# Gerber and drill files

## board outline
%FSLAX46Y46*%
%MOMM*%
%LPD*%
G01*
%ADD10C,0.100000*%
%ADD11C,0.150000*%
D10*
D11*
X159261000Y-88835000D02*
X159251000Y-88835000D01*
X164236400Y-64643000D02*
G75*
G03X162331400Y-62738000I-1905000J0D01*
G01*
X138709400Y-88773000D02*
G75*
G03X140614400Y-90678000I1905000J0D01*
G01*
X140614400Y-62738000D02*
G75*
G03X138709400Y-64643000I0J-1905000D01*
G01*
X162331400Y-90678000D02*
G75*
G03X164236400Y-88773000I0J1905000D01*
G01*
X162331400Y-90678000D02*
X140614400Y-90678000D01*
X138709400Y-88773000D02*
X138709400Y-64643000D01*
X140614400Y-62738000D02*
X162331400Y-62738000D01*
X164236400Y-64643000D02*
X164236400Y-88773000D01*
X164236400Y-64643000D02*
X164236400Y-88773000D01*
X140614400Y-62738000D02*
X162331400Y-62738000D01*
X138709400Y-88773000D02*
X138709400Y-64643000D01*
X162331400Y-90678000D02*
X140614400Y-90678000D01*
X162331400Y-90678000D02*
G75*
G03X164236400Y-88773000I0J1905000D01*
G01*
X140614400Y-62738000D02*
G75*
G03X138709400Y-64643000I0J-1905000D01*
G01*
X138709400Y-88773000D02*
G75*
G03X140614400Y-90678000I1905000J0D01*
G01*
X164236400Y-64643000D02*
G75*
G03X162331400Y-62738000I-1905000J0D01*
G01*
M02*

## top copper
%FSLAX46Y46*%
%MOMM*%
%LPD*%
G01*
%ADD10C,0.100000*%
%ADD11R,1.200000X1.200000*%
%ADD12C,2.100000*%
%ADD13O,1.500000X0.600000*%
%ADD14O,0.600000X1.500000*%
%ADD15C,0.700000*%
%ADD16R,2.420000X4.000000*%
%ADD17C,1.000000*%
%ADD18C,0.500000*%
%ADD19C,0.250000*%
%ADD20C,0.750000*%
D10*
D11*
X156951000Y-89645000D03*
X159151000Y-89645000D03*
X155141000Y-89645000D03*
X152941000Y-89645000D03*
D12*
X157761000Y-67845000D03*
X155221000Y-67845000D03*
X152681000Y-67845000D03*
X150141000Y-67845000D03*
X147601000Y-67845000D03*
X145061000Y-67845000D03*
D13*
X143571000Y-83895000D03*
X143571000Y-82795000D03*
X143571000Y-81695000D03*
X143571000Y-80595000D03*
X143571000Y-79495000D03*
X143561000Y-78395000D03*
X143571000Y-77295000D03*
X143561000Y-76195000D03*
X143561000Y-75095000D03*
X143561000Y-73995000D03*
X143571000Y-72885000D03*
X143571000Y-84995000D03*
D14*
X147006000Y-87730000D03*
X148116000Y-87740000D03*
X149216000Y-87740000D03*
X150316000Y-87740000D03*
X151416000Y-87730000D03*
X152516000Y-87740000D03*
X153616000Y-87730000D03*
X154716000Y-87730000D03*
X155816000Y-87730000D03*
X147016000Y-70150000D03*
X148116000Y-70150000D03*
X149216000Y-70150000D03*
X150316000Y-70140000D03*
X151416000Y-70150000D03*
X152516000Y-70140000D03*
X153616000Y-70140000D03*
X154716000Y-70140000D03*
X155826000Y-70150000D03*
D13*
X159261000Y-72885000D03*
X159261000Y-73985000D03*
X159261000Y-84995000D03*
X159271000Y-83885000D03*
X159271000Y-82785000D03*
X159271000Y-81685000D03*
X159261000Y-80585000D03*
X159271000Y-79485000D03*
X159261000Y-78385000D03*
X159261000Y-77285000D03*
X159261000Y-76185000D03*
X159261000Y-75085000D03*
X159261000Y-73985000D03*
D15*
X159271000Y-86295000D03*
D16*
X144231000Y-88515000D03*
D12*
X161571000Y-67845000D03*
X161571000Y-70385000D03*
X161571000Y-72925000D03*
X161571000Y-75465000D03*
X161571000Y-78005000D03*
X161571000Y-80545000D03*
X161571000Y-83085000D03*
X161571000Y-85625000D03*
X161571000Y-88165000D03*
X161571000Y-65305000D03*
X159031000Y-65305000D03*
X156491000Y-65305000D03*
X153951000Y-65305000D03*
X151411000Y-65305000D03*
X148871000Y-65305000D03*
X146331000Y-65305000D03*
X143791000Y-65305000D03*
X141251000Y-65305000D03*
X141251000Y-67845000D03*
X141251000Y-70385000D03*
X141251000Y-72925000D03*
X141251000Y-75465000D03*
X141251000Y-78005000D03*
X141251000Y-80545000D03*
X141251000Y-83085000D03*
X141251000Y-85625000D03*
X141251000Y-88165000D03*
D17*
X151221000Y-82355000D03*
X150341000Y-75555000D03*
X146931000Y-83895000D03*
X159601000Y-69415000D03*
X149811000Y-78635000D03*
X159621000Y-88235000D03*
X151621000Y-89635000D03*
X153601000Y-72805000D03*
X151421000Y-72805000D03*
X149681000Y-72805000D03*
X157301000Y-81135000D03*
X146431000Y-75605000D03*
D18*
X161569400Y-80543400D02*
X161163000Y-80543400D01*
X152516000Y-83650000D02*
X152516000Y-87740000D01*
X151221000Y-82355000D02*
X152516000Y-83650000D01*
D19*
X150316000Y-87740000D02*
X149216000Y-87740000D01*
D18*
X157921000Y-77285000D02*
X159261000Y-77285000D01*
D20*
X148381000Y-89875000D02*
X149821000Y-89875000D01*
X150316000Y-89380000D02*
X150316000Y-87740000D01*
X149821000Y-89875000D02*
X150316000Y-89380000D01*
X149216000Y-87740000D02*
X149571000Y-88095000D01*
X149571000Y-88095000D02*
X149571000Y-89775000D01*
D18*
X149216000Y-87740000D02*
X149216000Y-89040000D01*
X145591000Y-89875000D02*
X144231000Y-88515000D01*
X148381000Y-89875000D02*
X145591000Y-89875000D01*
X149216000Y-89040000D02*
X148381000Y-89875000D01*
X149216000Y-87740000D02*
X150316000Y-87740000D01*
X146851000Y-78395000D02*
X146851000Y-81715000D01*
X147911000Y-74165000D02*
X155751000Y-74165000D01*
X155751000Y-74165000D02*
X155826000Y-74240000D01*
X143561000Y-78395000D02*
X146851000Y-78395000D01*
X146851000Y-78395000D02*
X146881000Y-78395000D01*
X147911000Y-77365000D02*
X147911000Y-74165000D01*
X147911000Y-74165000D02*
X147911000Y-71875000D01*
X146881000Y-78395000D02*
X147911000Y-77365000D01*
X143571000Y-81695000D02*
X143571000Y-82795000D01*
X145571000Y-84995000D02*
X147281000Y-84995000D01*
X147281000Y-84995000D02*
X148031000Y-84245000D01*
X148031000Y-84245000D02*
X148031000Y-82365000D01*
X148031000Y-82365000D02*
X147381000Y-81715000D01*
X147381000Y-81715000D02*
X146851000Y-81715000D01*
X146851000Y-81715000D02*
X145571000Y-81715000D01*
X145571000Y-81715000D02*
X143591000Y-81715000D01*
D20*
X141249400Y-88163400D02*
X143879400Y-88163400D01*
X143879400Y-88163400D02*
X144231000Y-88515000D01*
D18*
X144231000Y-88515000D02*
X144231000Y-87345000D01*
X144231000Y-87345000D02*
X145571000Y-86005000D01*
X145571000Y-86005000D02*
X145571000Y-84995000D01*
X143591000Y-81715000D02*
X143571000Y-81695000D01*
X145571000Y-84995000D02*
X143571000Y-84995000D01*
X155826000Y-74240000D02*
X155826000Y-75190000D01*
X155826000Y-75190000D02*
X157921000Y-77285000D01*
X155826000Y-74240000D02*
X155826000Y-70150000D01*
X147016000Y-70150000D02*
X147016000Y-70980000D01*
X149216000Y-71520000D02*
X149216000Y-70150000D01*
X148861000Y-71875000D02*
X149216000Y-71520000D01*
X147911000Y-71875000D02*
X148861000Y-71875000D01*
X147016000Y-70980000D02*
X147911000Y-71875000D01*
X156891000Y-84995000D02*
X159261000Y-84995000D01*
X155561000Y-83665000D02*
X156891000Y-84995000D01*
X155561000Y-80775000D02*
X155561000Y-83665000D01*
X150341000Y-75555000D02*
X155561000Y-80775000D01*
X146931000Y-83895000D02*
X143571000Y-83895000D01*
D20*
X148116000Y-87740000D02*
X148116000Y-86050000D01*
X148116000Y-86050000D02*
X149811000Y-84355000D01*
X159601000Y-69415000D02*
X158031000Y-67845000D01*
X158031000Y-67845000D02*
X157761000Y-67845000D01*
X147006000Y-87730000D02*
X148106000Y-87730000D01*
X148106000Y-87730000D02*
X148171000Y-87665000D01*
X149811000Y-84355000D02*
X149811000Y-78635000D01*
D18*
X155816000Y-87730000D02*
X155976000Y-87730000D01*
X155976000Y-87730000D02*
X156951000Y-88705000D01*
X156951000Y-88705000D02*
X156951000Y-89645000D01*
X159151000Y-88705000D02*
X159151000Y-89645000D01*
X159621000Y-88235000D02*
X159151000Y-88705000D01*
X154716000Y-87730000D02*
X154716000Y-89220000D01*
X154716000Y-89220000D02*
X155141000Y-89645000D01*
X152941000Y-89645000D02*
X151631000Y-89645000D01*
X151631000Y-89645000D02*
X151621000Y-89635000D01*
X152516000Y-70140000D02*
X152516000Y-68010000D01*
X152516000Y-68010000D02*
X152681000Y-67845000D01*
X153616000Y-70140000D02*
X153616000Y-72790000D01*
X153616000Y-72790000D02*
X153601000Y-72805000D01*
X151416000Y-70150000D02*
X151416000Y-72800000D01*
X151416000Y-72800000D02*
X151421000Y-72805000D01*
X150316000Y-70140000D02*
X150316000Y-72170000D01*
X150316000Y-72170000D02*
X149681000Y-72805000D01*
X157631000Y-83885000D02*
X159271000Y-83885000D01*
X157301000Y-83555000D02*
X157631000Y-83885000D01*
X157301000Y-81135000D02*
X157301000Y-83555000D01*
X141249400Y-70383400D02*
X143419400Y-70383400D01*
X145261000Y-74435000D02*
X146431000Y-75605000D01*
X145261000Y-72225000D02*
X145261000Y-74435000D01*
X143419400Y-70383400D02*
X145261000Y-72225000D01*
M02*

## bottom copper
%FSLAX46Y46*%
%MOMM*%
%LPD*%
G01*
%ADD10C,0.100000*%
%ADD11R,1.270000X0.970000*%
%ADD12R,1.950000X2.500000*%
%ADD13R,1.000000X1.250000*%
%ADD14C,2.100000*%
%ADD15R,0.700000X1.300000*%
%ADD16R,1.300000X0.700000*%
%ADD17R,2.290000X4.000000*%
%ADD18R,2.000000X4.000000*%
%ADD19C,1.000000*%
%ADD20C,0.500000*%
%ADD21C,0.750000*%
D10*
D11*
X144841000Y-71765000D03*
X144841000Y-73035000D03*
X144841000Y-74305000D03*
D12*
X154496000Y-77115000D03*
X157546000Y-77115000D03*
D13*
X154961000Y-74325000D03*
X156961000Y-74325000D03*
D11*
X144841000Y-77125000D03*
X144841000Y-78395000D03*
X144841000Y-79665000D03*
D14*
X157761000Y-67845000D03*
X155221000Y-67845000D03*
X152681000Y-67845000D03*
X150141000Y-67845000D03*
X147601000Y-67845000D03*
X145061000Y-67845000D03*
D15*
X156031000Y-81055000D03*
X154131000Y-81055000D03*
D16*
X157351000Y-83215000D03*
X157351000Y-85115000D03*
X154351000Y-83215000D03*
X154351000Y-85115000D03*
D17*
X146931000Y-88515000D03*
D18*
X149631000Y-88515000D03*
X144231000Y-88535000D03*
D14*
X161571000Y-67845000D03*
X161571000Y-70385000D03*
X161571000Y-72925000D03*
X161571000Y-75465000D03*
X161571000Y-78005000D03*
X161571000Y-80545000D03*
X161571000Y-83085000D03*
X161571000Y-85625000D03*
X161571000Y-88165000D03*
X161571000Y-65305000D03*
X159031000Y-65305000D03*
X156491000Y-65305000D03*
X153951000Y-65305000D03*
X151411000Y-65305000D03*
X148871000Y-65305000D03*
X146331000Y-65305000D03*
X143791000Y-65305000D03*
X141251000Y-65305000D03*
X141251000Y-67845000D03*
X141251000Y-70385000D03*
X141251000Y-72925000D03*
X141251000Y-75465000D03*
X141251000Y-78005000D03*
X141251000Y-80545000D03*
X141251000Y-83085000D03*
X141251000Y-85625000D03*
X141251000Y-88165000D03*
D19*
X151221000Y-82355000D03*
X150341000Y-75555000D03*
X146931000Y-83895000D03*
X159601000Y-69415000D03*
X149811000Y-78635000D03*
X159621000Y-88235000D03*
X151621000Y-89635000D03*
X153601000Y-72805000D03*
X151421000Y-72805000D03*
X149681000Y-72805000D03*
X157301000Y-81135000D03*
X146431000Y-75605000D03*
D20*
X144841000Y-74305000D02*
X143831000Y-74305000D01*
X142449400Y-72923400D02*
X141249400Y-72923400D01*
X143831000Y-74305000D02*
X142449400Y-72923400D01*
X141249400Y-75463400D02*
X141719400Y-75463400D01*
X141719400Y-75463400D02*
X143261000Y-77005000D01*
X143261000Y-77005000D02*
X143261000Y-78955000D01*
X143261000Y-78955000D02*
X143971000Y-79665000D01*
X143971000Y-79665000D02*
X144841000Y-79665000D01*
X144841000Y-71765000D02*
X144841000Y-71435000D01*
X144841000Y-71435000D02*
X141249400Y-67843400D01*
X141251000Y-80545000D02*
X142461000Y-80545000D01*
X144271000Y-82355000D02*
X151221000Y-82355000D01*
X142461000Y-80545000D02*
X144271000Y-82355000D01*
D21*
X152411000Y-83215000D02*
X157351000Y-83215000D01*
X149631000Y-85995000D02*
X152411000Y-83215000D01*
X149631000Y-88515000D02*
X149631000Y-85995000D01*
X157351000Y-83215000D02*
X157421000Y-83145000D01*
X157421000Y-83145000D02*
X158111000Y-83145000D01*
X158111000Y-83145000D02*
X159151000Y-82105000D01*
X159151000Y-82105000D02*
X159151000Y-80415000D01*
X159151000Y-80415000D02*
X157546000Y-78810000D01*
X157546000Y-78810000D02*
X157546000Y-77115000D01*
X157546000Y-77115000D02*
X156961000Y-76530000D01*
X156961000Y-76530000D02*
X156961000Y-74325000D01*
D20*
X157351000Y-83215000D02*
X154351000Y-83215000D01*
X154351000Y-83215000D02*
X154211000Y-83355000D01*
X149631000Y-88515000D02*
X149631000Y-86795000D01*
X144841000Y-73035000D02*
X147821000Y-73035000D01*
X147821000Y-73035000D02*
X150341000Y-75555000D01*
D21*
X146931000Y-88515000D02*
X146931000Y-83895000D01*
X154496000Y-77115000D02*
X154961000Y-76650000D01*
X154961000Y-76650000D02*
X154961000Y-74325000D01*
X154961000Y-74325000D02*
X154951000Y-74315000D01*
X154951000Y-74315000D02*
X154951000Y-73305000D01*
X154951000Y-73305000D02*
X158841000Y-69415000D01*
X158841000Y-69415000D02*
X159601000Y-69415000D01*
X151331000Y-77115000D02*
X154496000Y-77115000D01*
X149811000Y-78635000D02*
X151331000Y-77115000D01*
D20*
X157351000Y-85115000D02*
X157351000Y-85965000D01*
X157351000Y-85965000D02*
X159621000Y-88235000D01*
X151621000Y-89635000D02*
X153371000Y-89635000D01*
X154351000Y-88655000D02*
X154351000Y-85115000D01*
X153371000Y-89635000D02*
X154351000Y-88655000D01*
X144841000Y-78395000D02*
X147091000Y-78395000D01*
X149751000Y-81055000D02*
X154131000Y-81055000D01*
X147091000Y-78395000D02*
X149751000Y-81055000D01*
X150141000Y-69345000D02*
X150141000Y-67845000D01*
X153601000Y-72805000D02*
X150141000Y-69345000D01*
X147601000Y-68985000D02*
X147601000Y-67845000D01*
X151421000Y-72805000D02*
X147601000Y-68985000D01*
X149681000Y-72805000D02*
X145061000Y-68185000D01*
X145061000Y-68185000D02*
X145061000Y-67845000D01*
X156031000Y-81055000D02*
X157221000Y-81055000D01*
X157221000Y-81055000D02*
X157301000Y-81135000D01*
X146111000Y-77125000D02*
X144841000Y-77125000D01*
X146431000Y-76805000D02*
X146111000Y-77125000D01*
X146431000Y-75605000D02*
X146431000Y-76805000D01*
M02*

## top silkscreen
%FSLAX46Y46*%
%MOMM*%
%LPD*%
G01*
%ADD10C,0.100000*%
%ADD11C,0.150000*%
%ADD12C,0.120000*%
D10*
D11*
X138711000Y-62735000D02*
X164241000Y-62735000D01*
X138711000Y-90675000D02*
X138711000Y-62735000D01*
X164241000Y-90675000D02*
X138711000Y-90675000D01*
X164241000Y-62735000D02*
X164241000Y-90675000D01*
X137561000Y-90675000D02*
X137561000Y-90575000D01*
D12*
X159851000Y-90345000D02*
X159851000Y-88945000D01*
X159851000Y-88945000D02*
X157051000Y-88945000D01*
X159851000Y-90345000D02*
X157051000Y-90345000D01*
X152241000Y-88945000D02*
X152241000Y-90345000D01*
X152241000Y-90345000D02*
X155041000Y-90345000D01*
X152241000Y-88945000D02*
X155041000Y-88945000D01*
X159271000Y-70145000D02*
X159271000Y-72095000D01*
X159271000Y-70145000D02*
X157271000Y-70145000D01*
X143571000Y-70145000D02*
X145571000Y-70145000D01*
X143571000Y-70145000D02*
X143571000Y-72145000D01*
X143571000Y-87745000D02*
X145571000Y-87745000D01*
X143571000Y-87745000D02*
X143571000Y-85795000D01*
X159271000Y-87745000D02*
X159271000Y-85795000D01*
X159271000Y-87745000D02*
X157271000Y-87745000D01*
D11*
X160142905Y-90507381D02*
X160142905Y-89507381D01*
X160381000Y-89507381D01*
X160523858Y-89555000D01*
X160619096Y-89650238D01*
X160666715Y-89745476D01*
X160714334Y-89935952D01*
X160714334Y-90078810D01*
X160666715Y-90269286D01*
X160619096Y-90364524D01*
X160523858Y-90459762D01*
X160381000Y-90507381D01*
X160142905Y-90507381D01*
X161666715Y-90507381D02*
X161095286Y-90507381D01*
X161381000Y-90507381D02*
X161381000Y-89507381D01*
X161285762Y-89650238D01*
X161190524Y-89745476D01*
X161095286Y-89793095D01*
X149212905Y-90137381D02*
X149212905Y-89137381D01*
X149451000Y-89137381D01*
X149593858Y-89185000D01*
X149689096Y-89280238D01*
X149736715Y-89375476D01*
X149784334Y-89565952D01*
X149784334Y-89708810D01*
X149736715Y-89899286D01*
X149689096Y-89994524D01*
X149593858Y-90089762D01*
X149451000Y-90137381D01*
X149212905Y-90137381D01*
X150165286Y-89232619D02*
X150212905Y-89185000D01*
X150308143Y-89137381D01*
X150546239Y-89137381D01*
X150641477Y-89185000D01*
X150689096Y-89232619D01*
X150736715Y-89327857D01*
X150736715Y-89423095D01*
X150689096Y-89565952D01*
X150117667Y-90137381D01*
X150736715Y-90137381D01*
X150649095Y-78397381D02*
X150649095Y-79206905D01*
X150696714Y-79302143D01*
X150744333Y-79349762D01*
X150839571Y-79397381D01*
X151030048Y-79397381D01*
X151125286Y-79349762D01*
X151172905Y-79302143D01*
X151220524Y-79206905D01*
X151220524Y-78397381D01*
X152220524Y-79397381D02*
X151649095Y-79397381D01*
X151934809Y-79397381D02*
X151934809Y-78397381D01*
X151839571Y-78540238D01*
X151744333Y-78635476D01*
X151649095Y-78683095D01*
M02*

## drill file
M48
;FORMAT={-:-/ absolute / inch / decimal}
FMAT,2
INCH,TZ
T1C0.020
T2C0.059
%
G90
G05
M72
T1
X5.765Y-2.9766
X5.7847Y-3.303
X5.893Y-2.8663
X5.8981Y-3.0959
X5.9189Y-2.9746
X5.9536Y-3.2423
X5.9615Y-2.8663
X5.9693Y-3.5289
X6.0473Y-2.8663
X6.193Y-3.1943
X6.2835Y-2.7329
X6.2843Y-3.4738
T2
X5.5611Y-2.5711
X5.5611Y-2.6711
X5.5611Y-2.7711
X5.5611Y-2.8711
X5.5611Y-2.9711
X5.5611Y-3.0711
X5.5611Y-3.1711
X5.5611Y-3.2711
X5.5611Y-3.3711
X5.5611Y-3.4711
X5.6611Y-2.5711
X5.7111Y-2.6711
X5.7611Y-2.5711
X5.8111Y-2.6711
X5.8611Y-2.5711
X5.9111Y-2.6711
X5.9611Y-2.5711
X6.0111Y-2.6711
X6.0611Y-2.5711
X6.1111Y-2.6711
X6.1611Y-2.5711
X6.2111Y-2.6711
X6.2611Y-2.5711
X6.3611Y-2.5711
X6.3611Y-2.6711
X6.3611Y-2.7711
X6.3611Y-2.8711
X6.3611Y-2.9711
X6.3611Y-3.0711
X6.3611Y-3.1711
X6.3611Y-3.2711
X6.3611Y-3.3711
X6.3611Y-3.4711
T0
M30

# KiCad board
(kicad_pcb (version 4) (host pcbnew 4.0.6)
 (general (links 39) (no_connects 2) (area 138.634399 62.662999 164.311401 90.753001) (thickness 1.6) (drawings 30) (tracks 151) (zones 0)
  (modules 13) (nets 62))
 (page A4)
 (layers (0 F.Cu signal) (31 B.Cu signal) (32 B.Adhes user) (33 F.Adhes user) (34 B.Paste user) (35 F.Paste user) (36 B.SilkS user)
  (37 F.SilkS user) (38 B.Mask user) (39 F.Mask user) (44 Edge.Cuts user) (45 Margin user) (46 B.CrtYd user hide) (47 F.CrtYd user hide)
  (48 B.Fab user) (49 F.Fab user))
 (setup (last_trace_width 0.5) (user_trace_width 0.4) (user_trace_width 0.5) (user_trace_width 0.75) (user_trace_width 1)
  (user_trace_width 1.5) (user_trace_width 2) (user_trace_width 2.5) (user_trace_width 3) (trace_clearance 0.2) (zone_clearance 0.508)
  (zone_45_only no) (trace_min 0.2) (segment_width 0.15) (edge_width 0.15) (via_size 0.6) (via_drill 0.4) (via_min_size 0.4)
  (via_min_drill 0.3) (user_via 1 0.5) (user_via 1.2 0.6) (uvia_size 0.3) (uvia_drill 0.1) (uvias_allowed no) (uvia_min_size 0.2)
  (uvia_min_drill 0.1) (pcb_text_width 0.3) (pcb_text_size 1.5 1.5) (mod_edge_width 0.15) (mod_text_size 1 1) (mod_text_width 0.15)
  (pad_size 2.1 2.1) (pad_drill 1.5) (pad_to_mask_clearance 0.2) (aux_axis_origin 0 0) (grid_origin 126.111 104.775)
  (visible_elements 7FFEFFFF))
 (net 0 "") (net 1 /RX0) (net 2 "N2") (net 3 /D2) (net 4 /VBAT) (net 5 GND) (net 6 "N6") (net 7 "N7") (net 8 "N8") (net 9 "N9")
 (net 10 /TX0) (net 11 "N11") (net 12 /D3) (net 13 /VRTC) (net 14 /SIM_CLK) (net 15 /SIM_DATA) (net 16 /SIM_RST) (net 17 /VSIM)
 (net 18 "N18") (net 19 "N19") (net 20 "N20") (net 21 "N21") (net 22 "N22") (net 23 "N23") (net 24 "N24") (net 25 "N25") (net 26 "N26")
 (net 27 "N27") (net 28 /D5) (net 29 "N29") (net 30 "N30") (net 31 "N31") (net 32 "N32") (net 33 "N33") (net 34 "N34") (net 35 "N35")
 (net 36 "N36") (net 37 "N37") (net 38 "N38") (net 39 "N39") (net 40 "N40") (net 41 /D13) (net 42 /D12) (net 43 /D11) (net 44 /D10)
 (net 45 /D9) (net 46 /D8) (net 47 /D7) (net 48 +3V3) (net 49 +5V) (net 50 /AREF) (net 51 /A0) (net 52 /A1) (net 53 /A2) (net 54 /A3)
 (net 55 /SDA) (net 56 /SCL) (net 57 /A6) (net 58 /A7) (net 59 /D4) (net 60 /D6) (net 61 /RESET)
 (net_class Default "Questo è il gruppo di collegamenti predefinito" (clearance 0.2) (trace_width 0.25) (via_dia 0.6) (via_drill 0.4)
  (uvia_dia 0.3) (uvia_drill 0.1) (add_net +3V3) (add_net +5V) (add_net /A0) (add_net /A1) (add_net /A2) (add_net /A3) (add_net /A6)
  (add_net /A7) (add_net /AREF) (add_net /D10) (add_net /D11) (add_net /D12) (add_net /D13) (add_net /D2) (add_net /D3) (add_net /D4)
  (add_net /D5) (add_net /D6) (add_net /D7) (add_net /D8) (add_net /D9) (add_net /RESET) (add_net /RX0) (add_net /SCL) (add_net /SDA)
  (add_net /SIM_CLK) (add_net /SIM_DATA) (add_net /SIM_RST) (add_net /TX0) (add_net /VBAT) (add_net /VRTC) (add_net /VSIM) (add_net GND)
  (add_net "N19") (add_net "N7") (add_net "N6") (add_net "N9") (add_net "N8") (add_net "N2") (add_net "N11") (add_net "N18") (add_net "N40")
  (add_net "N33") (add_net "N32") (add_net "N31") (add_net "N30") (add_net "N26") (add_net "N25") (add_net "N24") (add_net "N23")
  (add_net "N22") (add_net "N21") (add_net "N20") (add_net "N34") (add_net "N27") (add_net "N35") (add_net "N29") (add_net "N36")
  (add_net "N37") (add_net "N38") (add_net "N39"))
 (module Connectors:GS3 (layer B.Cu) (at 144.841 73.035 180)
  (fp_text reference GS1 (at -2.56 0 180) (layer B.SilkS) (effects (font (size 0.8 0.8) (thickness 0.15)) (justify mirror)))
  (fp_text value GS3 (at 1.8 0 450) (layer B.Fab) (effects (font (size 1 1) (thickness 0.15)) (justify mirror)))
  (pad 1 smd rect (at 0 1.27 180) (size 1.27 0.97) (layers B.Cu B.Paste B.Mask) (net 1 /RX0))
  (pad 2 smd rect (at 0 0 180) (size 1.27 0.97) (layers B.Cu B.Paste B.Mask) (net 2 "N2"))
  (pad 3 smd rect (at 0 -1.27 180) (size 1.27 0.97) (layers B.Cu B.Paste B.Mask) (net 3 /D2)))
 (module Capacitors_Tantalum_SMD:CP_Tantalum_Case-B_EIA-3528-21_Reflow (layer B.Cu) (at 156.021 77.115)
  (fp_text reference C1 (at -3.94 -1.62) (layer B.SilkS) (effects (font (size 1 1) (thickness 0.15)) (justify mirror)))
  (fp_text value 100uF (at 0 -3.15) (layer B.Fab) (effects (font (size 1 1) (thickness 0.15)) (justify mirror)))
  (pad 1 smd rect (at -1.525 0) (size 1.95 2.5) (layers B.Cu B.Paste B.Mask) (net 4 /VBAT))
  (pad 2 smd rect (at 1.525 0) (size 1.95 2.5) (layers B.Cu B.Paste B.Mask) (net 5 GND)))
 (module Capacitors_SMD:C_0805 (layer B.Cu) (at 155.961 74.325)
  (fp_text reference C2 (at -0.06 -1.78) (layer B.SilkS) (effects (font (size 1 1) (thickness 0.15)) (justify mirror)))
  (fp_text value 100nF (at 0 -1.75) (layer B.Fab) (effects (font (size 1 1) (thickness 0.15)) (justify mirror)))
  (pad 1 smd rect (at -1 0) (size 1 1.25) (layers B.Cu B.Paste B.Mask) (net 4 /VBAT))
  (pad 2 smd rect (at 1 0) (size 1 1.25) (layers B.Cu B.Paste B.Mask) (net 5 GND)))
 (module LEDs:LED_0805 (layer F.Cu) (at 158.051 89.645 180)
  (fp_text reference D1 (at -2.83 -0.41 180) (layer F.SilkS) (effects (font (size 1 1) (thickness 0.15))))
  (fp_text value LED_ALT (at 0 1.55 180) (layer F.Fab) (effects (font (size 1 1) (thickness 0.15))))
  (fp_line (start -1.8 -0.7) (end -1.8 0.7) (layer F.SilkS) (width 0.12))
  (fp_line (start -1.8 0.7) (end 1 0.7) (layer F.SilkS) (width 0.12))
  (fp_line (start -1.8 -0.7) (end 1 -0.7) (layer F.SilkS) (width 0.12))
  (pad 2 smd rect (at 1.1 0) (size 1.2 1.2) (layers F.Cu F.Paste F.Mask) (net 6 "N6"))
  (pad 1 smd rect (at -1.1 0) (size 1.2 1.2) (layers F.Cu F.Paste F.Mask) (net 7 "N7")))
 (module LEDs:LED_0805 (layer F.Cu) (at 154.041 89.645)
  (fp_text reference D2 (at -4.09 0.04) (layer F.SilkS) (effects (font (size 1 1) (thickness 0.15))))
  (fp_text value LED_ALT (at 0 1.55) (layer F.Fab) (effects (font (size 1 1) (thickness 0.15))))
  (fp_line (start -1.8 -0.7) (end -1.8 0.7) (layer F.SilkS) (width 0.12))
  (fp_line (start -1.8 0.7) (end 1 0.7) (layer F.SilkS) (width 0.12))
  (fp_line (start -1.8 -0.7) (end 1 -0.7) (layer F.SilkS) (width 0.12))
  (pad 2 smd rect (at 1.1 0 180) (size 1.2 1.2) (layers F.Cu F.Paste F.Mask) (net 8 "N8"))
  (pad 1 smd rect (at -1.1 0 180) (size 1.2 1.2) (layers F.Cu F.Paste F.Mask) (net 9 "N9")))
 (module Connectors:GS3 (layer B.Cu) (at 144.841 78.395 180)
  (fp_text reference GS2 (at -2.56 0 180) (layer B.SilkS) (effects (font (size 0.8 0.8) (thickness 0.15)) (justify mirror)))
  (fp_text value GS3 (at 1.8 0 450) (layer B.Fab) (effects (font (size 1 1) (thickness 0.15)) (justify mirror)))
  (pad 1 smd rect (at 0 1.27 180) (size 1.27 0.97) (layers B.Cu B.Paste B.Mask) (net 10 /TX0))
  (pad 2 smd rect (at 0 0 180) (size 1.27 0.97) (layers B.Cu B.Paste B.Mask) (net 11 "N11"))
  (pad 3 smd rect (at 0 -1.27 180) (size 1.27 0.97) (layers B.Cu B.Paste B.Mask) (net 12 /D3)))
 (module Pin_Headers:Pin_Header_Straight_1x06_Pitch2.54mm (layer B.Cu) (at 157.761 67.845 90)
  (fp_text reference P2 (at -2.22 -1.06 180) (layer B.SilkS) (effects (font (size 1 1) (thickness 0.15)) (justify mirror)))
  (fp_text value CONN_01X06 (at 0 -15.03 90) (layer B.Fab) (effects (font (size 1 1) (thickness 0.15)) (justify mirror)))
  (pad 1 thru_hole circle (at 0 0 90) (size 2.1 2.1) (drill 1.5) (layers *.Cu *.Mask) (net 4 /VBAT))
  (pad 2 thru_hole circle (at 0 -2.54 90) (size 2.1 2.1) (drill 1.5) (layers *.Cu *.Mask) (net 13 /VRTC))
  (pad 3 thru_hole circle (at 0 -5.08 90) (size 2.1 2.1) (drill 1.5) (layers *.Cu *.Mask) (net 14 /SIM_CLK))
  (pad 4 thru_hole circle (at 0 -7.62 90) (size 2.1 2.1) (drill 1.5) (layers *.Cu *.Mask) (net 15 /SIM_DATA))
  (pad 5 thru_hole circle (at 0 -10.16 90) (size 2.1 2.1) (drill 1.5) (layers *.Cu *.Mask) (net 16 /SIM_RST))
  (pad 6 thru_hole circle (at 0 -12.7 90) (size 2.1 2.1) (drill 1.5) (layers *.Cu *.Mask) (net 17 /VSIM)))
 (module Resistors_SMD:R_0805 (layer B.Cu) (at 155.081 81.055 180)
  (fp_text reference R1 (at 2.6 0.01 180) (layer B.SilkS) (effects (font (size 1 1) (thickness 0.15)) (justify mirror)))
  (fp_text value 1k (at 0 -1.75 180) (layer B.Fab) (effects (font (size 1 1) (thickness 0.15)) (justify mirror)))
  (pad 1 smd rect (at -0.95 0 180) (size 0.7 1.3) (layers B.Cu B.Paste B.Mask) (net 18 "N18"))
  (pad 2 smd rect (at 0.95 0 180) (size 0.7 1.3) (layers B.Cu B.Paste B.Mask) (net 11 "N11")))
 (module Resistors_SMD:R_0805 (layer B.Cu) (at 157.351 84.165 270)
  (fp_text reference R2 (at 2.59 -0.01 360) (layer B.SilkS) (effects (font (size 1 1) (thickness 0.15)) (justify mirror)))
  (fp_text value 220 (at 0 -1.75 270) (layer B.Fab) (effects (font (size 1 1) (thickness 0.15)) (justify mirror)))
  (pad 1 smd rect (at -0.95 0 270) (size 0.7 1.3) (layers B.Cu B.Paste B.Mask) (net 5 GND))
  (pad 2 smd rect (at 0.95 0 270) (size 0.7 1.3) (layers B.Cu B.Paste B.Mask) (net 7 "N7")))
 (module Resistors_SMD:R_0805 (layer B.Cu) (at 154.351 84.165 270)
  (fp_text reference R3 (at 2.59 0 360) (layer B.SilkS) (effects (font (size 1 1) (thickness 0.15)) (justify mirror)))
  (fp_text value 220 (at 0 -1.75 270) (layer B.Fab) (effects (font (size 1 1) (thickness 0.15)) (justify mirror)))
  (pad 1 smd rect (at -0.95 0 270) (size 0.7 1.3) (layers B.Cu B.Paste B.Mask) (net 5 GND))
  (pad 2 smd rect (at 0.95 0 270) (size 0.7 1.3) (layers B.Cu B.Paste B.Mask) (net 9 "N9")))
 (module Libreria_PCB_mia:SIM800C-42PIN (layer F.Cu) (at 151.421 78.945 180)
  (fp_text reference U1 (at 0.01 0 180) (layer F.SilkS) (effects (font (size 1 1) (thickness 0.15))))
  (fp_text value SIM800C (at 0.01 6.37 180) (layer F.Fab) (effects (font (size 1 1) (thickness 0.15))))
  (fp_line (start -7.85 8.8) (end -7.85 6.85) (layer F.SilkS) (width 0.12))
  (fp_line (start -7.85 8.8) (end -5.85 8.8) (layer F.SilkS) (width 0.12))
  (fp_line (start 7.85 8.8) (end 5.85 8.8) (layer F.SilkS) (width 0.12))
  (fp_line (start 7.85 8.8) (end 7.85 6.8) (layer F.SilkS) (width 0.12))
  (fp_line (start 7.85 -8.8) (end 5.85 -8.8) (layer F.SilkS) (width 0.12))
  (fp_line (start 7.85 -8.8) (end 7.85 -6.85) (layer F.SilkS) (width 0.12))
  (fp_line (start -7.85 -8.8) (end -7.85 -6.85) (layer F.SilkS) (width 0.12))
  (fp_line (start -7.85 -8.8) (end -5.85 -8.8) (layer F.SilkS) (width 0.12))
  (pad "" smd circle (at -7.85 -7.35 90) (size 0.7 0.7) (layers F.SilkS))
  (pad 32 smd oval (at 7.85 -4.95) (size 1.5 0.6) (layers F.Cu F.Paste F.Mask) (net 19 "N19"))
  (pad 31 smd oval (at 7.85 -3.85) (size 1.5 0.6) (layers F.Cu F.Paste F.Mask) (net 5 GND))
  (pad 30 smd oval (at 7.85 -2.75) (size 1.5 0.6) (layers F.Cu F.Paste F.Mask) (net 5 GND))
  (pad 29 smd oval (at 7.85 -1.65) (size 1.5 0.6) (layers F.Cu F.Paste F.Mask) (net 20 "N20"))
  (pad 28 smd oval (at 7.85 -0.55) (size 1.5 0.6) (layers F.Cu F.Paste F.Mask) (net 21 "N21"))
  (pad 27 smd oval (at 7.86 0.55) (size 1.5 0.6) (layers F.Cu F.Paste F.Mask) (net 5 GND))
  (pad 26 smd oval (at 7.85 1.65) (size 1.5 0.6) (layers F.Cu F.Paste F.Mask) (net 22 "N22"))
  (pad 25 smd oval (at 7.86 2.75) (size 1.5 0.6) (layers F.Cu F.Paste F.Mask) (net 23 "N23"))
  (pad 24 smd oval (at 7.86 3.85) (size 1.5 0.6) (layers F.Cu F.Paste F.Mask) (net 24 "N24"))
  (pad 23 smd oval (at 7.86 4.95) (size 1.5 0.6) (layers F.Cu F.Paste F.Mask) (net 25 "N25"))
  (pad 22 smd oval (at 7.85 6.06) (size 1.5 0.6) (layers F.Cu F.Paste F.Mask) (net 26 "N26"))
  (pad 33 smd oval (at 7.85 -6.05) (size 1.5 0.6) (layers F.Cu F.Paste F.Mask) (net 5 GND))
  (pad 34 smd oval (at 4.415 -8.785 90) (size 1.5 0.6) (layers F.Cu F.Paste F.Mask) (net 4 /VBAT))
  (pad 35 smd oval (at 3.305 -8.795 90) (size 1.5 0.6) (layers F.Cu F.Paste F.Mask) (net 4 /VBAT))
  (pad 36 smd oval (at 2.205 -8.795 90) (size 1.5 0.6) (layers F.Cu F.Paste F.Mask) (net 5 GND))
  (pad 37 smd oval (at 1.105 -8.795 90) (size 1.5 0.6) (layers F.Cu F.Paste F.Mask) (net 5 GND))
  (pad 38 smd oval (at 0.005 -8.785 90) (size 1.5 0.6) (layers F.Cu F.Paste F.Mask) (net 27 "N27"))
  (pad 39 smd oval (at -1.095 -8.795 90) (size 1.5 0.6) (layers F.Cu F.Paste F.Mask) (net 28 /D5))
  (pad 40 smd oval (at -2.195 -8.785 90) (size 1.5 0.6) (layers F.Cu F.Paste F.Mask) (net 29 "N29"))
  (pad 41 smd oval (at -3.295 -8.785 90) (size 1.5 0.6) (layers F.Cu F.Paste F.Mask) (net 8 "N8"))
  (pad 42 smd oval (at -4.395 -8.785 90) (size 1.5 0.6) (layers F.Cu F.Paste F.Mask) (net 6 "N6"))
  (pad 21 smd oval (at 4.405 8.795 270) (size 1.5 0.6) (layers F.Cu F.Paste F.Mask) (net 5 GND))
  (pad 20 smd oval (at 3.305 8.795 270) (size 1.5 0.6) (layers F.Cu F.Paste F.Mask) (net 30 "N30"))
  (pad 19 smd oval (at 2.205 8.795 270) (size 1.5 0.6) (layers F.Cu F.Paste F.Mask) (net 5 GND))
  (pad 18 smd oval (at 1.105 8.805 270) (size 1.5 0.6) (layers F.Cu F.Paste F.Mask) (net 17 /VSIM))
  (pad 17 smd oval (at 0.005 8.795 270) (size 1.5 0.6) (layers F.Cu F.Paste F.Mask) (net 16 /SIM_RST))
  (pad 16 smd oval (at -1.095 8.805 270) (size 1.5 0.6) (layers F.Cu F.Paste F.Mask) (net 14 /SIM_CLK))
  (pad 15 smd oval (at -2.195 8.805 270) (size 1.5 0.6) (layers F.Cu F.Paste F.Mask) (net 15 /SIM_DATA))
  (pad 14 smd oval (at -3.295 8.805 270) (size 1.5 0.6) (layers F.Cu F.Paste F.Mask) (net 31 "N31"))
  (pad 13 smd oval (at -4.405 8.795 270) (size 1.5 0.6) (layers F.Cu F.Paste F.Mask) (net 5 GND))
  (pad 12 smd oval (at -7.84 6.06 180) (size 1.5 0.6) (layers F.Cu F.Paste F.Mask) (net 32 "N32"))
  (pad 11 smd oval (at -7.84 4.96 180) (size 1.5 0.6) (layers F.Cu F.Paste F.Mask) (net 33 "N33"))
  (pad 1 smd oval (at -7.84 -6.05 180) (size 1.5 0.6) (layers F.Cu F.Paste F.Mask) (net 2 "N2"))
  (pad 2 smd oval (at -7.85 -4.94 180) (size 1.5 0.6) (layers F.Cu F.Paste F.Mask) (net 18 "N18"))
  (pad 3 smd oval (at -7.85 -3.84 180) (size 1.5 0.6) (layers F.Cu F.Paste F.Mask) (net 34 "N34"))
  (pad 4 smd oval (at -7.85 -2.74 180) (size 1.5 0.6) (layers F.Cu F.Paste F.Mask) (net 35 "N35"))
  (pad 5 smd oval (at -7.84 -1.64 180) (size 1.5 0.6) (layers F.Cu F.Paste F.Mask) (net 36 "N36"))
  (pad 6 smd oval (at -7.85 -0.54 180) (size 1.5 0.6) (layers F.Cu F.Paste F.Mask) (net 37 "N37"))
  (pad 7 smd oval (at -7.84 0.56 180) (size 1.5 0.6) (layers F.Cu F.Paste F.Mask) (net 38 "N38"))
  (pad 8 smd oval (at -7.84 1.66 180) (size 1.5 0.6) (layers F.Cu F.Paste F.Mask) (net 5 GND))
  (pad 9 smd oval (at -7.84 2.76 180) (size 1.5 0.6) (layers F.Cu F.Paste F.Mask) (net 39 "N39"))
  (pad 10 smd oval (at -7.84 3.86 180) (size 1.5 0.6) (layers F.Cu F.Paste F.Mask) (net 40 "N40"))
  (pad 11 smd oval (at -7.84 4.96 180) (size 1.5 0.6) (layers F.Cu F.Paste F.Mask) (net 33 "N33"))
  (pad "" smd circle (at -7.85 -7.35 90) (size 0.7 0.7) (layers F.Cu F.Paste F.Mask)))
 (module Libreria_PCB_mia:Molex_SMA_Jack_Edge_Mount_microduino (layer B.Cu) (at 146.931 88.535 90)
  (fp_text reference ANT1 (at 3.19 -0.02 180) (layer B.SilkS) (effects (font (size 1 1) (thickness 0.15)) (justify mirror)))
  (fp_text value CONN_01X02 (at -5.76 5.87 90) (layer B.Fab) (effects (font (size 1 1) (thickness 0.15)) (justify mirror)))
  (pad 1 smd rect (at 0.02 0 90) (size 4 2.29) (layers B.Cu B.Paste B.Mask) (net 19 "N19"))
  (pad 2 smd rect (at 0.02 2.7 90) (size 4 2) (layers B.Cu B.Paste B.Mask) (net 5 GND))
  (pad 2 smd rect (at 0 -2.7 90) (size 4 2) (layers B.Cu B.Paste B.Mask) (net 5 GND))
  (pad 2 smd rect (at 0.02 -2.7 90) (size 4 2.42) (layers F.Cu F.Paste F.Mask) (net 5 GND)))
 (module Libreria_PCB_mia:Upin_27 (layer B.Cu) (at 161.571 88.165 180)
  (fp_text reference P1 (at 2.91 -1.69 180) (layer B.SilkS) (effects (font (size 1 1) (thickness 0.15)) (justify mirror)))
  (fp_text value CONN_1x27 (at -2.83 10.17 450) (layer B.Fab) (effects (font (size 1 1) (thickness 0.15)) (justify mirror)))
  (pad 9 thru_hole circle (at 0 20.32 180) (size 2.1 2.1) (drill 1.5) (layers *.Cu *.Mask) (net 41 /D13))
  (pad 8 thru_hole circle (at 0 17.78 180) (size 2.1 2.1) (drill 1.5) (layers *.Cu *.Mask) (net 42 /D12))
  (pad 7 thru_hole circle (at 0 15.24 180) (size 2.1 2.1) (drill 1.5) (layers *.Cu *.Mask) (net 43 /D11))
  (pad 6 thru_hole circle (at 0 12.7 180) (size 2.1 2.1) (drill 1.5) (layers *.Cu *.Mask) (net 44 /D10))
  (pad 5 thru_hole circle (at 0 10.16 180) (size 2.1 2.1) (drill 1.5) (layers *.Cu *.Mask) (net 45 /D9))
  (pad 4 thru_hole circle (at 0 7.62 180) (size 2.1 2.1) (drill 1.5) (layers *.Cu *.Mask) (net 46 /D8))
  (pad 3 thru_hole circle (at 0 5.08 180) (size 2.1 2.1) (drill 1.5) (layers *.Cu *.Mask) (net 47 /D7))
  (pad 2 thru_hole circle (at 0 2.54 180) (size 2.1 2.1) (drill 1.5) (layers *.Cu *.Mask) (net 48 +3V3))
  (pad 1 thru_hole circle (at 0 0 180) (size 2.1 2.1) (drill 1.5) (layers *.Cu *.Mask) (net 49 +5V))
  (pad 10 thru_hole circle (at 0 22.86 180) (size 2.1 2.1) (drill 1.5) (layers *.Cu *.Mask) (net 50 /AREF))
  (pad 11 thru_hole circle (at 2.54 22.86 180) (size 2.1 2.1) (drill 1.5) (layers *.Cu *.Mask) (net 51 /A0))
  (pad 12 thru_hole circle (at 5.08 22.86 180) (size 2.1 2.1) (drill 1.5) (layers *.Cu *.Mask) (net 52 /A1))
  (pad 13 thru_hole circle (at 7.62 22.86 180) (size 2.1 2.1) (drill 1.5) (layers *.Cu *.Mask) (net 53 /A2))
  (pad 14 thru_hole circle (at 10.16 22.86 180) (size 2.1 2.1) (drill 1.5) (layers *.Cu *.Mask) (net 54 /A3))
  (pad 15 thru_hole circle (at 12.7 22.86 180) (size 2.1 2.1) (drill 1.5) (layers *.Cu *.Mask) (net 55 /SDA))
  (pad 16 thru_hole circle (at 15.24 22.86 180) (size 2.1 2.1) (drill 1.5) (layers *.Cu *.Mask) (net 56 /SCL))
  (pad 17 thru_hole circle (at 17.78 22.86 180) (size 2.1 2.1) (drill 1.5) (layers *.Cu *.Mask) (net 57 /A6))
  (pad 18 thru_hole circle (at 20.32 22.86 180) (size 2.1 2.1) (drill 1.5) (layers *.Cu *.Mask) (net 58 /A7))
  (pad 19 thru_hole circle (at 20.32 20.32 180) (size 2.1 2.1) (drill 1.5) (layers *.Cu *.Mask) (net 1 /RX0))
  (pad 20 thru_hole circle (at 20.32 17.78 180) (size 2.1 2.1) (drill 1.5) (layers *.Cu *.Mask) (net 10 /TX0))
  (pad 21 thru_hole circle (at 20.32 15.24 180) (size 2.1 2.1) (drill 1.5) (layers *.Cu *.Mask) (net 3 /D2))
  (pad 22 thru_hole circle (at 20.32 12.7 180) (size 2.1 2.1) (drill 1.5) (layers *.Cu *.Mask) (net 12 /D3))
  (pad 23 thru_hole circle (at 20.32 10.16 180) (size 2.1 2.1) (drill 1.5) (layers *.Cu *.Mask) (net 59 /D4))
  (pad 24 thru_hole circle (at 20.32 7.62 180) (size 2.1 2.1) (drill 1.5) (layers *.Cu *.Mask) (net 28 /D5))
  (pad 25 thru_hole circle (at 20.32 5.08 180) (size 2.1 2.1) (drill 1.5) (layers *.Cu *.Mask) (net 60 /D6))
  (pad 26 thru_hole circle (at 20.32 2.54 180) (size 2.1 2.1) (drill 1.5) (layers *.Cu *.Mask) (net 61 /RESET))
  (pad 27 thru_hole circle (at 20.32 0 180) (size 2.1 2.1) (drill 1.5) (layers *.Cu *.Mask) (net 5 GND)))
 (gr_line (start 138.711 62.735) (end 164.241 62.735) (angle 90) (layer F.SilkS) (width 0.15))
 (gr_line (start 138.711 90.675) (end 138.711 62.735) (angle 90) (layer F.SilkS) (width 0.15))
 (gr_line (start 164.241 90.675) (end 138.711 90.675) (angle 90) (layer F.SilkS) (width 0.15))
 (gr_line (start 164.241 62.735) (end 164.241 90.675) (angle 90) (layer F.SilkS) (width 0.15))
 (gr_line (start 137.561 90.675) (end 137.561 90.575) (angle 90) (layer F.SilkS) (width 0.15))
 (gr_line (start 159.261 88.835) (end 159.251 88.835) (angle 90) (layer Edge.Cuts) (width 0.15))
 (gr_arc (start 162.3314 64.643) (end 162.3314 62.738) (angle 90) (layer Edge.Cuts) (width 0.15))
 (gr_arc (start 140.6144 88.773) (end 140.6144 90.678) (angle 90) (layer Edge.Cuts) (width 0.15))
 (gr_arc (start 140.6144 64.643) (end 138.7094 64.643) (angle 90) (layer Edge.Cuts) (width 0.15))
 (gr_arc (start 162.3314 88.773) (end 164.2364 88.773) (angle 90) (layer Edge.Cuts) (width 0.15))
 (gr_line (start 162.3314 90.678) (end 140.6144 90.678) (angle 90) (layer Edge.Cuts) (width 0.15))
 (gr_line (start 138.7094 88.773) (end 138.7094 64.643) (angle 90) (layer Edge.Cuts) (width 0.15))
 (gr_line (start 140.6144 62.738) (end 162.3314 62.738) (angle 90) (layer Edge.Cuts) (width 0.15))
 (gr_line (start 164.2364 64.643) (end 164.2364 88.773) (angle 90) (layer Edge.Cuts) (width 0.15))
 (gr_line (start 164.2364 64.643) (end 164.2364 88.773) (angle 90) (layer Edge.Cuts) (width 0.15))
 (gr_line (start 140.6144 62.738) (end 162.3314 62.738) (angle 90) (layer Edge.Cuts) (width 0.15))
 (gr_line (start 138.7094 88.773) (end 138.7094 64.643) (angle 90) (layer Edge.Cuts) (width 0.15))
 (gr_line (start 162.3314 90.678) (end 140.6144 90.678) (angle 90) (layer Edge.Cuts) (width 0.15))
 (gr_arc (start 162.3314 88.773) (end 164.2364 88.773) (angle 90) (layer Edge.Cuts) (width 0.15))
 (gr_arc (start 140.6144 64.643) (end 138.7094 64.643) (angle 90) (layer Edge.Cuts) (width 0.15))
 (gr_arc (start 140.6144 88.773) (end 140.6144 90.678) (angle 90) (layer Edge.Cuts) (width 0.15))
 (gr_arc (start 162.3314 64.643) (end 162.3314 62.738) (angle 90) (layer Edge.Cuts) (width 0.15))
 (segment (start 161.5694 80.5434) (end 161.163 80.5434) (width 0.5) (layer F.Cu) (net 46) (status 30))
 (segment (start 144.841 74.305) (end 143.831 74.305) (width 0.5) (layer B.Cu) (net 3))
 (segment (start 142.4494 72.9234) (end 141.2494 72.9234) (width 0.5) (layer B.Cu) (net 3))
 (segment (start 143.831 74.305) (end 142.4494 72.9234) (width 0.5) (layer B.Cu) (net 3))
 (segment (start 141.2494 75.4634) (end 141.7194 75.4634) (width 0.5) (layer B.Cu) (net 12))
 (segment (start 141.7194 75.4634) (end 143.261 77.005) (width 0.5) (layer B.Cu) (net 12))
 (segment (start 143.261 77.005) (end 143.261 78.955) (width 0.5) (layer B.Cu) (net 12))
 (segment (start 143.261 78.955) (end 143.971 79.665) (width 0.5) (layer B.Cu) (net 12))
 (segment (start 143.971 79.665) (end 144.841 79.665) (width 0.5) (layer B.Cu) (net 12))
 (segment (start 144.841 71.765) (end 144.841 71.435) (width 0.5) (layer B.Cu) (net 1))
 (segment (start 144.841 71.435) (end 141.2494 67.8434) (width 0.5) (layer B.Cu) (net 1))
 (segment (start 141.251 80.545) (end 142.461 80.545) (width 0.5) (layer B.Cu) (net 28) (status 400000))
 (via (at 151.221 82.355) (size 1) (drill 0.5) (layers F.Cu B.Cu) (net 28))
 (segment (start 152.516 83.65) (end 152.516 87.74) (width 0.5) (layer F.Cu) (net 28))
 (segment (start 151.221 82.355) (end 152.516 83.65) (width 0.5) (layer F.Cu) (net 28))
 (segment (start 144.271 82.355) (end 151.221 82.355) (width 0.5) (layer B.Cu) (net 28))
 (segment (start 142.461 80.545) (end 144.271 82.355) (width 0.5) (layer B.Cu) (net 28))
 (segment (start 150.316 87.74) (end 149.216 87.74) (width 0.25) (layer F.Cu) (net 5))
 (segment (start 152.411 83.215) (end 157.351 83.215) (width 0.75) (layer B.Cu) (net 5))
 (segment (start 149.631 85.995) (end 152.411 83.215) (width 0.75) (layer B.Cu) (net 5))
 (segment (start 157.921 77.285) (end 159.261 77.285) (width 0.5) (layer F.Cu) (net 5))
 (segment (start 148.381 89.875) (end 149.821 89.875) (width 0.75) (layer F.Cu) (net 5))
 (segment (start 150.316 89.38) (end 150.316 87.74) (width 0.75) (layer F.Cu) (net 5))
 (segment (start 149.821 89.875) (end 150.316 89.38) (width 0.75) (layer F.Cu) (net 5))
 (segment (start 149.216 87.74) (end 149.571 88.095) (width 0.75) (layer F.Cu) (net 5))
 (segment (start 149.571 88.095) (end 149.571 89.775) (width 0.75) (layer F.Cu) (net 5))
 (segment (start 149.216 87.74) (end 149.216 89.04) (width 0.5) (layer F.Cu) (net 5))
 (segment (start 145.591 89.875) (end 144.231 88.515) (width 0.5) (layer F.Cu) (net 5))
 (segment (start 148.381 89.875) (end 145.591 89.875) (width 0.5) (layer F.Cu) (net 5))
 (segment (start 149.216 89.04) (end 148.381 89.875) (width 0.5) (layer F.Cu) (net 5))
 (segment (start 149.216 87.74) (end 150.316 87.74) (width 0.5) (layer F.Cu) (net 5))
 (segment (start 146.851 78.395) (end 146.851 81.715) (width 0.5) (layer F.Cu) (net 5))
 (segment (start 147.911 74.165) (end 155.751 74.165) (width 0.5) (layer F.Cu) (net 5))
 (segment (start 155.751 74.165) (end 155.826 74.24) (width 0.5) (layer F.Cu) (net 5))
 (segment (start 143.561 78.395) (end 146.851 78.395) (width 0.5) (layer F.Cu) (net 5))
 (segment (start 146.851 78.395) (end 146.881 78.395) (width 0.5) (layer F.Cu) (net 5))
 (segment (start 147.911 77.365) (end 147.911 74.165) (width 0.5) (layer F.Cu) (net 5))
 (segment (start 147.911 74.165) (end 147.911 71.875) (width 0.5) (layer F.Cu) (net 5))
 (segment (start 146.881 78.395) (end 147.911 77.365) (width 0.5) (layer F.Cu) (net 5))
 (segment (start 149.631 88.515) (end 149.631 85.995) (width 0.75) (layer B.Cu) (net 5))
 (segment (start 157.351 83.215) (end 157.421 83.145) (width 0.75) (layer B.Cu) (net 5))
 (segment (start 157.421 83.145) (end 158.111 83.145) (width 0.75) (layer B.Cu) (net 5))
 (segment (start 158.111 83.145) (end 159.151 82.105) (width 0.75) (layer B.Cu) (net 5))
 (segment (start 159.151 82.105) (end 159.151 80.415) (width 0.75) (layer B.Cu) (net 5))
 (segment (start 159.151 80.415) (end 157.546 78.81) (width 0.75) (layer B.Cu) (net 5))
 (segment (start 157.546 78.81) (end 157.546 77.115) (width 0.75) (layer B.Cu) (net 5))
 (segment (start 157.546 77.115) (end 156.961 76.53) (width 0.75) (layer B.Cu) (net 5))
 (segment (start 156.961 76.53) (end 156.961 74.325) (width 0.75) (layer B.Cu) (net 5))
 (segment (start 143.571 81.695) (end 143.571 82.795) (width 0.5) (layer F.Cu) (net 5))
 (segment (start 145.571 84.995) (end 147.281 84.995) (width 0.5) (layer F.Cu) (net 5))
 (segment (start 147.281 84.995) (end 148.031 84.245) (width 0.5) (layer F.Cu) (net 5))
 (segment (start 148.031 84.245) (end 148.031 82.365) (width 0.5) (layer F.Cu) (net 5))
 (segment (start 148.031 82.365) (end 147.381 81.715) (width 0.5) (layer F.Cu) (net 5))
 (segment (start 147.381 81.715) (end 146.851 81.715) (width 0.5) (layer F.Cu) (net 5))
 (segment (start 146.851 81.715) (end 145.571 81.715) (width 0.5) (layer F.Cu) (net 5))
 (segment (start 145.571 81.715) (end 143.591 81.715) (width 0.5) (layer F.Cu) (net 5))
 (segment (start 141.2494 88.1634) (end 143.8794 88.1634) (width 0.75) (layer F.Cu) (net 5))
 (segment (start 143.8794 88.1634) (end 144.231 88.515) (width 0.75) (layer F.Cu) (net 5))
 (segment (start 157.351 83.215) (end 154.351 83.215) (width 0.5) (layer B.Cu) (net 5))
 (segment (start 154.351 83.215) (end 154.211 83.355) (width 0.5) (layer B.Cu) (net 5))
 (segment (start 144.231 88.515) (end 144.231 87.345) (width 0.5) (layer F.Cu) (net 5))
 (segment (start 144.231 87.345) (end 145.571 86.005) (width 0.5) (layer F.Cu) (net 5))
 (segment (start 145.571 86.005) (end 145.571 84.995) (width 0.5) (layer F.Cu) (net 5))
 (segment (start 143.591 81.715) (end 143.571 81.695) (width 0.5) (layer F.Cu) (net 5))
 (segment (start 145.571 84.995) (end 143.571 84.995) (width 0.5) (layer F.Cu) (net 5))
 (segment (start 155.826 74.24) (end 155.826 75.19) (width 0.5) (layer F.Cu) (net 5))
 (segment (start 155.826 75.19) (end 157.921 77.285) (width 0.5) (layer F.Cu) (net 5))
 (segment (start 155.826 74.24) (end 155.826 70.15) (width 0.5) (layer F.Cu) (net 5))
 (segment (start 147.016 70.15) (end 147.016 70.98) (width 0.5) (layer F.Cu) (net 5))
 (segment (start 149.216 71.52) (end 149.216 70.15) (width 0.5) (layer F.Cu) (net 5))
 (segment (start 148.861 71.875) (end 149.216 71.52) (width 0.5) (layer F.Cu) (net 5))
 (segment (start 147.911 71.875) (end 148.861 71.875) (width 0.5) (layer F.Cu) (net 5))
 (segment (start 147.016 70.98) (end 147.911 71.875) (width 0.5) (layer F.Cu) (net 5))
 (segment (start 149.631 88.515) (end 149.631 86.795) (width 0.5) (layer B.Cu) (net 5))
 (segment (start 144.841 73.035) (end 147.821 73.035) (width 0.5) (layer B.Cu) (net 2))
 (segment (start 156.891 84.995) (end 159.261 84.995) (width 0.5) (layer F.Cu) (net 2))
 (segment (start 155.561 83.665) (end 156.891 84.995) (width 0.5) (layer F.Cu) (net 2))
 (segment (start 155.561 80.775) (end 155.561 83.665) (width 0.5) (layer F.Cu) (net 2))
 (segment (start 150.341 75.555) (end 155.561 80.775) (width 0.5) (layer F.Cu) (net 2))
 (via (at 150.341 75.555) (size 1) (drill 0.5) (layers F.Cu B.Cu) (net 2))
 (segment (start 147.821 73.035) (end 150.341 75.555) (width 0.5) (layer B.Cu) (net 2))
 (segment (start 146.931 88.515) (end 146.931 83.895) (width 0.75) (layer B.Cu) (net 19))
 (segment (start 146.931 83.895) (end 143.571 83.895) (width 0.5) (layer F.Cu) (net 19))
 (via (at 146.931 83.895) (size 1) (drill 0.5) (layers F.Cu B.Cu) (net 19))
 (segment (start 154.496 77.115) (end 154.961 76.65) (width 0.75) (layer B.Cu) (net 4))
 (segment (start 148.116 87.74) (end 148.116 86.05) (width 0.75) (layer F.Cu) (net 4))
 (segment (start 148.116 86.05) (end 149.811 84.355) (width 0.75) (layer F.Cu) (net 4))
 (segment (start 154.961 76.65) (end 154.961 74.325) (width 0.75) (layer B.Cu) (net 4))
 (segment (start 154.961 74.325) (end 154.951 74.315) (width 0.75) (layer B.Cu) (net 4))
 (segment (start 154.951 74.315) (end 154.951 73.305) (width 0.75) (layer B.Cu) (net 4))
 (segment (start 154.951 73.305) (end 158.841 69.415) (width 0.75) (layer B.Cu) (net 4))
 (segment (start 158.841 69.415) (end 159.601 69.415) (width 0.75) (layer B.Cu) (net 4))
 (via (at 159.601 69.415) (size 1) (drill 0.5) (layers F.Cu B.Cu) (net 4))
 (segment (start 159.601 69.415) (end 158.031 67.845) (width 0.75) (layer F.Cu) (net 4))
 (segment (start 158.031 67.845) (end 157.761 67.845) (width 0.75) (layer F.Cu) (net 4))
 (segment (start 147.006 87.73) (end 148.106 87.73) (width 0.75) (layer F.Cu) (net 4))
 (segment (start 148.106 87.73) (end 148.171 87.665) (width 0.75) (layer F.Cu) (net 4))
 (segment (start 151.331 77.115) (end 154.496 77.115) (width 0.75) (layer B.Cu) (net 4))
 (segment (start 149.811 78.635) (end 151.331 77.115) (width 0.75) (layer B.Cu) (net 4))
 (via (at 149.811 78.635) (size 1) (drill 0.5) (layers F.Cu B.Cu) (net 4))
 (segment (start 149.811 84.355) (end 149.811 78.635) (width 0.75) (layer F.Cu) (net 4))
 (segment (start 155.816 87.73) (end 155.976 87.73) (width 0.5) (layer F.Cu) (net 6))
 (segment (start 155.976 87.73) (end 156.951 88.705) (width 0.5) (layer F.Cu) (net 6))
 (segment (start 156.951 88.705) (end 156.951 89.645) (width 0.5) (layer F.Cu) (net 6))
 (segment (start 157.351 85.115) (end 157.351 85.965) (width 0.5) (layer B.Cu) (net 7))
 (segment (start 159.151 88.705) (end 159.151 89.645) (width 0.5) (layer F.Cu) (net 7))
 (segment (start 159.621 88.235) (end 159.151 88.705) (width 0.5) (layer F.Cu) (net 7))
 (via (at 159.621 88.235) (size 1) (drill 0.5) (layers F.Cu B.Cu) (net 7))
 (segment (start 157.351 85.965) (end 159.621 88.235) (width 0.5) (layer B.Cu) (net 7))
 (segment (start 154.716 87.73) (end 154.716 89.22) (width 0.5) (layer F.Cu) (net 8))
 (segment (start 154.716 89.22) (end 155.141 89.645) (width 0.5) (layer F.Cu) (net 8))
 (segment (start 152.941 89.645) (end 151.631 89.645) (width 0.5) (layer F.Cu) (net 9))
 (segment (start 151.621 89.635) (end 153.371 89.635) (width 0.5) (layer B.Cu) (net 9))
 (via (at 151.621 89.635) (size 1) (drill 0.5) (layers F.Cu B.Cu) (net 9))
 (segment (start 151.631 89.645) (end 151.621 89.635) (width 0.5) (layer F.Cu) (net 9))
 (segment (start 154.351 88.655) (end 154.351 85.115) (width 0.5) (layer B.Cu) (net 9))
 (segment (start 153.371 89.635) (end 154.351 88.655) (width 0.5) (layer B.Cu) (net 9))
 (segment (start 144.841 78.395) (end 147.091 78.395) (width 0.5) (layer B.Cu) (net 11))
 (segment (start 149.751 81.055) (end 154.131 81.055) (width 0.5) (layer B.Cu) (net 11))
 (segment (start 147.091 78.395) (end 149.751 81.055) (width 0.5) (layer B.Cu) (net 11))
 (segment (start 152.516 70.14) (end 152.516 68.01) (width 0.5) (layer F.Cu) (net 14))
 (segment (start 152.516 68.01) (end 152.681 67.845) (width 0.5) (layer F.Cu) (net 14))
 (segment (start 153.616 70.14) (end 153.616 72.79) (width 0.5) (layer F.Cu) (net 15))
 (segment (start 150.141 69.345) (end 150.141 67.845) (width 0.5) (layer B.Cu) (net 15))
 (segment (start 153.601 72.805) (end 150.141 69.345) (width 0.5) (layer B.Cu) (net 15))
 (via (at 153.601 72.805) (size 1) (drill 0.5) (layers F.Cu B.Cu) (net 15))
 (segment (start 153.616 72.79) (end 153.601 72.805) (width 0.5) (layer F.Cu) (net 15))
 (segment (start 151.416 70.15) (end 151.416 72.8) (width 0.5) (layer F.Cu) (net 16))
 (segment (start 147.601 68.985) (end 147.601 67.845) (width 0.5) (layer B.Cu) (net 16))
 (segment (start 151.421 72.805) (end 147.601 68.985) (width 0.5) (layer B.Cu) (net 16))
 (via (at 151.421 72.805) (size 1) (drill 0.5) (layers F.Cu B.Cu) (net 16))
 (segment (start 151.416 72.8) (end 151.421 72.805) (width 0.5) (layer F.Cu) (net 16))
 (segment (start 150.316 70.14) (end 150.316 72.17) (width 0.5) (layer F.Cu) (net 17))
 (segment (start 149.681 72.805) (end 145.061 68.185) (width 0.5) (layer B.Cu) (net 17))
 (via (at 149.681 72.805) (size 1) (drill 0.5) (layers F.Cu B.Cu) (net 17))
 (segment (start 150.316 72.17) (end 149.681 72.805) (width 0.5) (layer F.Cu) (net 17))
 (segment (start 145.061 68.185) (end 145.061 67.845) (width 0.5) (layer B.Cu) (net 17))
 (segment (start 156.031 81.055) (end 157.221 81.055) (width 0.5) (layer B.Cu) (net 18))
 (segment (start 157.631 83.885) (end 159.271 83.885) (width 0.5) (layer F.Cu) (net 18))
 (segment (start 157.301 83.555) (end 157.631 83.885) (width 0.5) (layer F.Cu) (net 18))
 (segment (start 157.301 81.135) (end 157.301 83.555) (width 0.5) (layer F.Cu) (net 18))
 (via (at 157.301 81.135) (size 1) (drill 0.5) (layers F.Cu B.Cu) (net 18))
 (segment (start 157.221 81.055) (end 157.301 81.135) (width 0.5) (layer B.Cu) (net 18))
 (segment (start 141.2494 70.3834) (end 143.4194 70.3834) (width 0.5) (layer F.Cu) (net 10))
 (segment (start 146.111 77.125) (end 144.841 77.125) (width 0.5) (layer B.Cu) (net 10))
 (segment (start 146.431 76.805) (end 146.111 77.125) (width 0.5) (layer B.Cu) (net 10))
 (segment (start 146.431 75.605) (end 146.431 76.805) (width 0.5) (layer B.Cu) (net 10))
 (via (at 146.431 75.605) (size 1) (drill 0.5) (layers F.Cu B.Cu) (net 10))
 (segment (start 145.261 74.435) (end 146.431 75.605) (width 0.5) (layer F.Cu) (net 10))
 (segment (start 145.261 72.225) (end 145.261 74.435) (width 0.5) (layer F.Cu) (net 10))
 (segment (start 143.4194 70.3834) (end 145.261 72.225) (width 0.5) (layer F.Cu) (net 10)))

